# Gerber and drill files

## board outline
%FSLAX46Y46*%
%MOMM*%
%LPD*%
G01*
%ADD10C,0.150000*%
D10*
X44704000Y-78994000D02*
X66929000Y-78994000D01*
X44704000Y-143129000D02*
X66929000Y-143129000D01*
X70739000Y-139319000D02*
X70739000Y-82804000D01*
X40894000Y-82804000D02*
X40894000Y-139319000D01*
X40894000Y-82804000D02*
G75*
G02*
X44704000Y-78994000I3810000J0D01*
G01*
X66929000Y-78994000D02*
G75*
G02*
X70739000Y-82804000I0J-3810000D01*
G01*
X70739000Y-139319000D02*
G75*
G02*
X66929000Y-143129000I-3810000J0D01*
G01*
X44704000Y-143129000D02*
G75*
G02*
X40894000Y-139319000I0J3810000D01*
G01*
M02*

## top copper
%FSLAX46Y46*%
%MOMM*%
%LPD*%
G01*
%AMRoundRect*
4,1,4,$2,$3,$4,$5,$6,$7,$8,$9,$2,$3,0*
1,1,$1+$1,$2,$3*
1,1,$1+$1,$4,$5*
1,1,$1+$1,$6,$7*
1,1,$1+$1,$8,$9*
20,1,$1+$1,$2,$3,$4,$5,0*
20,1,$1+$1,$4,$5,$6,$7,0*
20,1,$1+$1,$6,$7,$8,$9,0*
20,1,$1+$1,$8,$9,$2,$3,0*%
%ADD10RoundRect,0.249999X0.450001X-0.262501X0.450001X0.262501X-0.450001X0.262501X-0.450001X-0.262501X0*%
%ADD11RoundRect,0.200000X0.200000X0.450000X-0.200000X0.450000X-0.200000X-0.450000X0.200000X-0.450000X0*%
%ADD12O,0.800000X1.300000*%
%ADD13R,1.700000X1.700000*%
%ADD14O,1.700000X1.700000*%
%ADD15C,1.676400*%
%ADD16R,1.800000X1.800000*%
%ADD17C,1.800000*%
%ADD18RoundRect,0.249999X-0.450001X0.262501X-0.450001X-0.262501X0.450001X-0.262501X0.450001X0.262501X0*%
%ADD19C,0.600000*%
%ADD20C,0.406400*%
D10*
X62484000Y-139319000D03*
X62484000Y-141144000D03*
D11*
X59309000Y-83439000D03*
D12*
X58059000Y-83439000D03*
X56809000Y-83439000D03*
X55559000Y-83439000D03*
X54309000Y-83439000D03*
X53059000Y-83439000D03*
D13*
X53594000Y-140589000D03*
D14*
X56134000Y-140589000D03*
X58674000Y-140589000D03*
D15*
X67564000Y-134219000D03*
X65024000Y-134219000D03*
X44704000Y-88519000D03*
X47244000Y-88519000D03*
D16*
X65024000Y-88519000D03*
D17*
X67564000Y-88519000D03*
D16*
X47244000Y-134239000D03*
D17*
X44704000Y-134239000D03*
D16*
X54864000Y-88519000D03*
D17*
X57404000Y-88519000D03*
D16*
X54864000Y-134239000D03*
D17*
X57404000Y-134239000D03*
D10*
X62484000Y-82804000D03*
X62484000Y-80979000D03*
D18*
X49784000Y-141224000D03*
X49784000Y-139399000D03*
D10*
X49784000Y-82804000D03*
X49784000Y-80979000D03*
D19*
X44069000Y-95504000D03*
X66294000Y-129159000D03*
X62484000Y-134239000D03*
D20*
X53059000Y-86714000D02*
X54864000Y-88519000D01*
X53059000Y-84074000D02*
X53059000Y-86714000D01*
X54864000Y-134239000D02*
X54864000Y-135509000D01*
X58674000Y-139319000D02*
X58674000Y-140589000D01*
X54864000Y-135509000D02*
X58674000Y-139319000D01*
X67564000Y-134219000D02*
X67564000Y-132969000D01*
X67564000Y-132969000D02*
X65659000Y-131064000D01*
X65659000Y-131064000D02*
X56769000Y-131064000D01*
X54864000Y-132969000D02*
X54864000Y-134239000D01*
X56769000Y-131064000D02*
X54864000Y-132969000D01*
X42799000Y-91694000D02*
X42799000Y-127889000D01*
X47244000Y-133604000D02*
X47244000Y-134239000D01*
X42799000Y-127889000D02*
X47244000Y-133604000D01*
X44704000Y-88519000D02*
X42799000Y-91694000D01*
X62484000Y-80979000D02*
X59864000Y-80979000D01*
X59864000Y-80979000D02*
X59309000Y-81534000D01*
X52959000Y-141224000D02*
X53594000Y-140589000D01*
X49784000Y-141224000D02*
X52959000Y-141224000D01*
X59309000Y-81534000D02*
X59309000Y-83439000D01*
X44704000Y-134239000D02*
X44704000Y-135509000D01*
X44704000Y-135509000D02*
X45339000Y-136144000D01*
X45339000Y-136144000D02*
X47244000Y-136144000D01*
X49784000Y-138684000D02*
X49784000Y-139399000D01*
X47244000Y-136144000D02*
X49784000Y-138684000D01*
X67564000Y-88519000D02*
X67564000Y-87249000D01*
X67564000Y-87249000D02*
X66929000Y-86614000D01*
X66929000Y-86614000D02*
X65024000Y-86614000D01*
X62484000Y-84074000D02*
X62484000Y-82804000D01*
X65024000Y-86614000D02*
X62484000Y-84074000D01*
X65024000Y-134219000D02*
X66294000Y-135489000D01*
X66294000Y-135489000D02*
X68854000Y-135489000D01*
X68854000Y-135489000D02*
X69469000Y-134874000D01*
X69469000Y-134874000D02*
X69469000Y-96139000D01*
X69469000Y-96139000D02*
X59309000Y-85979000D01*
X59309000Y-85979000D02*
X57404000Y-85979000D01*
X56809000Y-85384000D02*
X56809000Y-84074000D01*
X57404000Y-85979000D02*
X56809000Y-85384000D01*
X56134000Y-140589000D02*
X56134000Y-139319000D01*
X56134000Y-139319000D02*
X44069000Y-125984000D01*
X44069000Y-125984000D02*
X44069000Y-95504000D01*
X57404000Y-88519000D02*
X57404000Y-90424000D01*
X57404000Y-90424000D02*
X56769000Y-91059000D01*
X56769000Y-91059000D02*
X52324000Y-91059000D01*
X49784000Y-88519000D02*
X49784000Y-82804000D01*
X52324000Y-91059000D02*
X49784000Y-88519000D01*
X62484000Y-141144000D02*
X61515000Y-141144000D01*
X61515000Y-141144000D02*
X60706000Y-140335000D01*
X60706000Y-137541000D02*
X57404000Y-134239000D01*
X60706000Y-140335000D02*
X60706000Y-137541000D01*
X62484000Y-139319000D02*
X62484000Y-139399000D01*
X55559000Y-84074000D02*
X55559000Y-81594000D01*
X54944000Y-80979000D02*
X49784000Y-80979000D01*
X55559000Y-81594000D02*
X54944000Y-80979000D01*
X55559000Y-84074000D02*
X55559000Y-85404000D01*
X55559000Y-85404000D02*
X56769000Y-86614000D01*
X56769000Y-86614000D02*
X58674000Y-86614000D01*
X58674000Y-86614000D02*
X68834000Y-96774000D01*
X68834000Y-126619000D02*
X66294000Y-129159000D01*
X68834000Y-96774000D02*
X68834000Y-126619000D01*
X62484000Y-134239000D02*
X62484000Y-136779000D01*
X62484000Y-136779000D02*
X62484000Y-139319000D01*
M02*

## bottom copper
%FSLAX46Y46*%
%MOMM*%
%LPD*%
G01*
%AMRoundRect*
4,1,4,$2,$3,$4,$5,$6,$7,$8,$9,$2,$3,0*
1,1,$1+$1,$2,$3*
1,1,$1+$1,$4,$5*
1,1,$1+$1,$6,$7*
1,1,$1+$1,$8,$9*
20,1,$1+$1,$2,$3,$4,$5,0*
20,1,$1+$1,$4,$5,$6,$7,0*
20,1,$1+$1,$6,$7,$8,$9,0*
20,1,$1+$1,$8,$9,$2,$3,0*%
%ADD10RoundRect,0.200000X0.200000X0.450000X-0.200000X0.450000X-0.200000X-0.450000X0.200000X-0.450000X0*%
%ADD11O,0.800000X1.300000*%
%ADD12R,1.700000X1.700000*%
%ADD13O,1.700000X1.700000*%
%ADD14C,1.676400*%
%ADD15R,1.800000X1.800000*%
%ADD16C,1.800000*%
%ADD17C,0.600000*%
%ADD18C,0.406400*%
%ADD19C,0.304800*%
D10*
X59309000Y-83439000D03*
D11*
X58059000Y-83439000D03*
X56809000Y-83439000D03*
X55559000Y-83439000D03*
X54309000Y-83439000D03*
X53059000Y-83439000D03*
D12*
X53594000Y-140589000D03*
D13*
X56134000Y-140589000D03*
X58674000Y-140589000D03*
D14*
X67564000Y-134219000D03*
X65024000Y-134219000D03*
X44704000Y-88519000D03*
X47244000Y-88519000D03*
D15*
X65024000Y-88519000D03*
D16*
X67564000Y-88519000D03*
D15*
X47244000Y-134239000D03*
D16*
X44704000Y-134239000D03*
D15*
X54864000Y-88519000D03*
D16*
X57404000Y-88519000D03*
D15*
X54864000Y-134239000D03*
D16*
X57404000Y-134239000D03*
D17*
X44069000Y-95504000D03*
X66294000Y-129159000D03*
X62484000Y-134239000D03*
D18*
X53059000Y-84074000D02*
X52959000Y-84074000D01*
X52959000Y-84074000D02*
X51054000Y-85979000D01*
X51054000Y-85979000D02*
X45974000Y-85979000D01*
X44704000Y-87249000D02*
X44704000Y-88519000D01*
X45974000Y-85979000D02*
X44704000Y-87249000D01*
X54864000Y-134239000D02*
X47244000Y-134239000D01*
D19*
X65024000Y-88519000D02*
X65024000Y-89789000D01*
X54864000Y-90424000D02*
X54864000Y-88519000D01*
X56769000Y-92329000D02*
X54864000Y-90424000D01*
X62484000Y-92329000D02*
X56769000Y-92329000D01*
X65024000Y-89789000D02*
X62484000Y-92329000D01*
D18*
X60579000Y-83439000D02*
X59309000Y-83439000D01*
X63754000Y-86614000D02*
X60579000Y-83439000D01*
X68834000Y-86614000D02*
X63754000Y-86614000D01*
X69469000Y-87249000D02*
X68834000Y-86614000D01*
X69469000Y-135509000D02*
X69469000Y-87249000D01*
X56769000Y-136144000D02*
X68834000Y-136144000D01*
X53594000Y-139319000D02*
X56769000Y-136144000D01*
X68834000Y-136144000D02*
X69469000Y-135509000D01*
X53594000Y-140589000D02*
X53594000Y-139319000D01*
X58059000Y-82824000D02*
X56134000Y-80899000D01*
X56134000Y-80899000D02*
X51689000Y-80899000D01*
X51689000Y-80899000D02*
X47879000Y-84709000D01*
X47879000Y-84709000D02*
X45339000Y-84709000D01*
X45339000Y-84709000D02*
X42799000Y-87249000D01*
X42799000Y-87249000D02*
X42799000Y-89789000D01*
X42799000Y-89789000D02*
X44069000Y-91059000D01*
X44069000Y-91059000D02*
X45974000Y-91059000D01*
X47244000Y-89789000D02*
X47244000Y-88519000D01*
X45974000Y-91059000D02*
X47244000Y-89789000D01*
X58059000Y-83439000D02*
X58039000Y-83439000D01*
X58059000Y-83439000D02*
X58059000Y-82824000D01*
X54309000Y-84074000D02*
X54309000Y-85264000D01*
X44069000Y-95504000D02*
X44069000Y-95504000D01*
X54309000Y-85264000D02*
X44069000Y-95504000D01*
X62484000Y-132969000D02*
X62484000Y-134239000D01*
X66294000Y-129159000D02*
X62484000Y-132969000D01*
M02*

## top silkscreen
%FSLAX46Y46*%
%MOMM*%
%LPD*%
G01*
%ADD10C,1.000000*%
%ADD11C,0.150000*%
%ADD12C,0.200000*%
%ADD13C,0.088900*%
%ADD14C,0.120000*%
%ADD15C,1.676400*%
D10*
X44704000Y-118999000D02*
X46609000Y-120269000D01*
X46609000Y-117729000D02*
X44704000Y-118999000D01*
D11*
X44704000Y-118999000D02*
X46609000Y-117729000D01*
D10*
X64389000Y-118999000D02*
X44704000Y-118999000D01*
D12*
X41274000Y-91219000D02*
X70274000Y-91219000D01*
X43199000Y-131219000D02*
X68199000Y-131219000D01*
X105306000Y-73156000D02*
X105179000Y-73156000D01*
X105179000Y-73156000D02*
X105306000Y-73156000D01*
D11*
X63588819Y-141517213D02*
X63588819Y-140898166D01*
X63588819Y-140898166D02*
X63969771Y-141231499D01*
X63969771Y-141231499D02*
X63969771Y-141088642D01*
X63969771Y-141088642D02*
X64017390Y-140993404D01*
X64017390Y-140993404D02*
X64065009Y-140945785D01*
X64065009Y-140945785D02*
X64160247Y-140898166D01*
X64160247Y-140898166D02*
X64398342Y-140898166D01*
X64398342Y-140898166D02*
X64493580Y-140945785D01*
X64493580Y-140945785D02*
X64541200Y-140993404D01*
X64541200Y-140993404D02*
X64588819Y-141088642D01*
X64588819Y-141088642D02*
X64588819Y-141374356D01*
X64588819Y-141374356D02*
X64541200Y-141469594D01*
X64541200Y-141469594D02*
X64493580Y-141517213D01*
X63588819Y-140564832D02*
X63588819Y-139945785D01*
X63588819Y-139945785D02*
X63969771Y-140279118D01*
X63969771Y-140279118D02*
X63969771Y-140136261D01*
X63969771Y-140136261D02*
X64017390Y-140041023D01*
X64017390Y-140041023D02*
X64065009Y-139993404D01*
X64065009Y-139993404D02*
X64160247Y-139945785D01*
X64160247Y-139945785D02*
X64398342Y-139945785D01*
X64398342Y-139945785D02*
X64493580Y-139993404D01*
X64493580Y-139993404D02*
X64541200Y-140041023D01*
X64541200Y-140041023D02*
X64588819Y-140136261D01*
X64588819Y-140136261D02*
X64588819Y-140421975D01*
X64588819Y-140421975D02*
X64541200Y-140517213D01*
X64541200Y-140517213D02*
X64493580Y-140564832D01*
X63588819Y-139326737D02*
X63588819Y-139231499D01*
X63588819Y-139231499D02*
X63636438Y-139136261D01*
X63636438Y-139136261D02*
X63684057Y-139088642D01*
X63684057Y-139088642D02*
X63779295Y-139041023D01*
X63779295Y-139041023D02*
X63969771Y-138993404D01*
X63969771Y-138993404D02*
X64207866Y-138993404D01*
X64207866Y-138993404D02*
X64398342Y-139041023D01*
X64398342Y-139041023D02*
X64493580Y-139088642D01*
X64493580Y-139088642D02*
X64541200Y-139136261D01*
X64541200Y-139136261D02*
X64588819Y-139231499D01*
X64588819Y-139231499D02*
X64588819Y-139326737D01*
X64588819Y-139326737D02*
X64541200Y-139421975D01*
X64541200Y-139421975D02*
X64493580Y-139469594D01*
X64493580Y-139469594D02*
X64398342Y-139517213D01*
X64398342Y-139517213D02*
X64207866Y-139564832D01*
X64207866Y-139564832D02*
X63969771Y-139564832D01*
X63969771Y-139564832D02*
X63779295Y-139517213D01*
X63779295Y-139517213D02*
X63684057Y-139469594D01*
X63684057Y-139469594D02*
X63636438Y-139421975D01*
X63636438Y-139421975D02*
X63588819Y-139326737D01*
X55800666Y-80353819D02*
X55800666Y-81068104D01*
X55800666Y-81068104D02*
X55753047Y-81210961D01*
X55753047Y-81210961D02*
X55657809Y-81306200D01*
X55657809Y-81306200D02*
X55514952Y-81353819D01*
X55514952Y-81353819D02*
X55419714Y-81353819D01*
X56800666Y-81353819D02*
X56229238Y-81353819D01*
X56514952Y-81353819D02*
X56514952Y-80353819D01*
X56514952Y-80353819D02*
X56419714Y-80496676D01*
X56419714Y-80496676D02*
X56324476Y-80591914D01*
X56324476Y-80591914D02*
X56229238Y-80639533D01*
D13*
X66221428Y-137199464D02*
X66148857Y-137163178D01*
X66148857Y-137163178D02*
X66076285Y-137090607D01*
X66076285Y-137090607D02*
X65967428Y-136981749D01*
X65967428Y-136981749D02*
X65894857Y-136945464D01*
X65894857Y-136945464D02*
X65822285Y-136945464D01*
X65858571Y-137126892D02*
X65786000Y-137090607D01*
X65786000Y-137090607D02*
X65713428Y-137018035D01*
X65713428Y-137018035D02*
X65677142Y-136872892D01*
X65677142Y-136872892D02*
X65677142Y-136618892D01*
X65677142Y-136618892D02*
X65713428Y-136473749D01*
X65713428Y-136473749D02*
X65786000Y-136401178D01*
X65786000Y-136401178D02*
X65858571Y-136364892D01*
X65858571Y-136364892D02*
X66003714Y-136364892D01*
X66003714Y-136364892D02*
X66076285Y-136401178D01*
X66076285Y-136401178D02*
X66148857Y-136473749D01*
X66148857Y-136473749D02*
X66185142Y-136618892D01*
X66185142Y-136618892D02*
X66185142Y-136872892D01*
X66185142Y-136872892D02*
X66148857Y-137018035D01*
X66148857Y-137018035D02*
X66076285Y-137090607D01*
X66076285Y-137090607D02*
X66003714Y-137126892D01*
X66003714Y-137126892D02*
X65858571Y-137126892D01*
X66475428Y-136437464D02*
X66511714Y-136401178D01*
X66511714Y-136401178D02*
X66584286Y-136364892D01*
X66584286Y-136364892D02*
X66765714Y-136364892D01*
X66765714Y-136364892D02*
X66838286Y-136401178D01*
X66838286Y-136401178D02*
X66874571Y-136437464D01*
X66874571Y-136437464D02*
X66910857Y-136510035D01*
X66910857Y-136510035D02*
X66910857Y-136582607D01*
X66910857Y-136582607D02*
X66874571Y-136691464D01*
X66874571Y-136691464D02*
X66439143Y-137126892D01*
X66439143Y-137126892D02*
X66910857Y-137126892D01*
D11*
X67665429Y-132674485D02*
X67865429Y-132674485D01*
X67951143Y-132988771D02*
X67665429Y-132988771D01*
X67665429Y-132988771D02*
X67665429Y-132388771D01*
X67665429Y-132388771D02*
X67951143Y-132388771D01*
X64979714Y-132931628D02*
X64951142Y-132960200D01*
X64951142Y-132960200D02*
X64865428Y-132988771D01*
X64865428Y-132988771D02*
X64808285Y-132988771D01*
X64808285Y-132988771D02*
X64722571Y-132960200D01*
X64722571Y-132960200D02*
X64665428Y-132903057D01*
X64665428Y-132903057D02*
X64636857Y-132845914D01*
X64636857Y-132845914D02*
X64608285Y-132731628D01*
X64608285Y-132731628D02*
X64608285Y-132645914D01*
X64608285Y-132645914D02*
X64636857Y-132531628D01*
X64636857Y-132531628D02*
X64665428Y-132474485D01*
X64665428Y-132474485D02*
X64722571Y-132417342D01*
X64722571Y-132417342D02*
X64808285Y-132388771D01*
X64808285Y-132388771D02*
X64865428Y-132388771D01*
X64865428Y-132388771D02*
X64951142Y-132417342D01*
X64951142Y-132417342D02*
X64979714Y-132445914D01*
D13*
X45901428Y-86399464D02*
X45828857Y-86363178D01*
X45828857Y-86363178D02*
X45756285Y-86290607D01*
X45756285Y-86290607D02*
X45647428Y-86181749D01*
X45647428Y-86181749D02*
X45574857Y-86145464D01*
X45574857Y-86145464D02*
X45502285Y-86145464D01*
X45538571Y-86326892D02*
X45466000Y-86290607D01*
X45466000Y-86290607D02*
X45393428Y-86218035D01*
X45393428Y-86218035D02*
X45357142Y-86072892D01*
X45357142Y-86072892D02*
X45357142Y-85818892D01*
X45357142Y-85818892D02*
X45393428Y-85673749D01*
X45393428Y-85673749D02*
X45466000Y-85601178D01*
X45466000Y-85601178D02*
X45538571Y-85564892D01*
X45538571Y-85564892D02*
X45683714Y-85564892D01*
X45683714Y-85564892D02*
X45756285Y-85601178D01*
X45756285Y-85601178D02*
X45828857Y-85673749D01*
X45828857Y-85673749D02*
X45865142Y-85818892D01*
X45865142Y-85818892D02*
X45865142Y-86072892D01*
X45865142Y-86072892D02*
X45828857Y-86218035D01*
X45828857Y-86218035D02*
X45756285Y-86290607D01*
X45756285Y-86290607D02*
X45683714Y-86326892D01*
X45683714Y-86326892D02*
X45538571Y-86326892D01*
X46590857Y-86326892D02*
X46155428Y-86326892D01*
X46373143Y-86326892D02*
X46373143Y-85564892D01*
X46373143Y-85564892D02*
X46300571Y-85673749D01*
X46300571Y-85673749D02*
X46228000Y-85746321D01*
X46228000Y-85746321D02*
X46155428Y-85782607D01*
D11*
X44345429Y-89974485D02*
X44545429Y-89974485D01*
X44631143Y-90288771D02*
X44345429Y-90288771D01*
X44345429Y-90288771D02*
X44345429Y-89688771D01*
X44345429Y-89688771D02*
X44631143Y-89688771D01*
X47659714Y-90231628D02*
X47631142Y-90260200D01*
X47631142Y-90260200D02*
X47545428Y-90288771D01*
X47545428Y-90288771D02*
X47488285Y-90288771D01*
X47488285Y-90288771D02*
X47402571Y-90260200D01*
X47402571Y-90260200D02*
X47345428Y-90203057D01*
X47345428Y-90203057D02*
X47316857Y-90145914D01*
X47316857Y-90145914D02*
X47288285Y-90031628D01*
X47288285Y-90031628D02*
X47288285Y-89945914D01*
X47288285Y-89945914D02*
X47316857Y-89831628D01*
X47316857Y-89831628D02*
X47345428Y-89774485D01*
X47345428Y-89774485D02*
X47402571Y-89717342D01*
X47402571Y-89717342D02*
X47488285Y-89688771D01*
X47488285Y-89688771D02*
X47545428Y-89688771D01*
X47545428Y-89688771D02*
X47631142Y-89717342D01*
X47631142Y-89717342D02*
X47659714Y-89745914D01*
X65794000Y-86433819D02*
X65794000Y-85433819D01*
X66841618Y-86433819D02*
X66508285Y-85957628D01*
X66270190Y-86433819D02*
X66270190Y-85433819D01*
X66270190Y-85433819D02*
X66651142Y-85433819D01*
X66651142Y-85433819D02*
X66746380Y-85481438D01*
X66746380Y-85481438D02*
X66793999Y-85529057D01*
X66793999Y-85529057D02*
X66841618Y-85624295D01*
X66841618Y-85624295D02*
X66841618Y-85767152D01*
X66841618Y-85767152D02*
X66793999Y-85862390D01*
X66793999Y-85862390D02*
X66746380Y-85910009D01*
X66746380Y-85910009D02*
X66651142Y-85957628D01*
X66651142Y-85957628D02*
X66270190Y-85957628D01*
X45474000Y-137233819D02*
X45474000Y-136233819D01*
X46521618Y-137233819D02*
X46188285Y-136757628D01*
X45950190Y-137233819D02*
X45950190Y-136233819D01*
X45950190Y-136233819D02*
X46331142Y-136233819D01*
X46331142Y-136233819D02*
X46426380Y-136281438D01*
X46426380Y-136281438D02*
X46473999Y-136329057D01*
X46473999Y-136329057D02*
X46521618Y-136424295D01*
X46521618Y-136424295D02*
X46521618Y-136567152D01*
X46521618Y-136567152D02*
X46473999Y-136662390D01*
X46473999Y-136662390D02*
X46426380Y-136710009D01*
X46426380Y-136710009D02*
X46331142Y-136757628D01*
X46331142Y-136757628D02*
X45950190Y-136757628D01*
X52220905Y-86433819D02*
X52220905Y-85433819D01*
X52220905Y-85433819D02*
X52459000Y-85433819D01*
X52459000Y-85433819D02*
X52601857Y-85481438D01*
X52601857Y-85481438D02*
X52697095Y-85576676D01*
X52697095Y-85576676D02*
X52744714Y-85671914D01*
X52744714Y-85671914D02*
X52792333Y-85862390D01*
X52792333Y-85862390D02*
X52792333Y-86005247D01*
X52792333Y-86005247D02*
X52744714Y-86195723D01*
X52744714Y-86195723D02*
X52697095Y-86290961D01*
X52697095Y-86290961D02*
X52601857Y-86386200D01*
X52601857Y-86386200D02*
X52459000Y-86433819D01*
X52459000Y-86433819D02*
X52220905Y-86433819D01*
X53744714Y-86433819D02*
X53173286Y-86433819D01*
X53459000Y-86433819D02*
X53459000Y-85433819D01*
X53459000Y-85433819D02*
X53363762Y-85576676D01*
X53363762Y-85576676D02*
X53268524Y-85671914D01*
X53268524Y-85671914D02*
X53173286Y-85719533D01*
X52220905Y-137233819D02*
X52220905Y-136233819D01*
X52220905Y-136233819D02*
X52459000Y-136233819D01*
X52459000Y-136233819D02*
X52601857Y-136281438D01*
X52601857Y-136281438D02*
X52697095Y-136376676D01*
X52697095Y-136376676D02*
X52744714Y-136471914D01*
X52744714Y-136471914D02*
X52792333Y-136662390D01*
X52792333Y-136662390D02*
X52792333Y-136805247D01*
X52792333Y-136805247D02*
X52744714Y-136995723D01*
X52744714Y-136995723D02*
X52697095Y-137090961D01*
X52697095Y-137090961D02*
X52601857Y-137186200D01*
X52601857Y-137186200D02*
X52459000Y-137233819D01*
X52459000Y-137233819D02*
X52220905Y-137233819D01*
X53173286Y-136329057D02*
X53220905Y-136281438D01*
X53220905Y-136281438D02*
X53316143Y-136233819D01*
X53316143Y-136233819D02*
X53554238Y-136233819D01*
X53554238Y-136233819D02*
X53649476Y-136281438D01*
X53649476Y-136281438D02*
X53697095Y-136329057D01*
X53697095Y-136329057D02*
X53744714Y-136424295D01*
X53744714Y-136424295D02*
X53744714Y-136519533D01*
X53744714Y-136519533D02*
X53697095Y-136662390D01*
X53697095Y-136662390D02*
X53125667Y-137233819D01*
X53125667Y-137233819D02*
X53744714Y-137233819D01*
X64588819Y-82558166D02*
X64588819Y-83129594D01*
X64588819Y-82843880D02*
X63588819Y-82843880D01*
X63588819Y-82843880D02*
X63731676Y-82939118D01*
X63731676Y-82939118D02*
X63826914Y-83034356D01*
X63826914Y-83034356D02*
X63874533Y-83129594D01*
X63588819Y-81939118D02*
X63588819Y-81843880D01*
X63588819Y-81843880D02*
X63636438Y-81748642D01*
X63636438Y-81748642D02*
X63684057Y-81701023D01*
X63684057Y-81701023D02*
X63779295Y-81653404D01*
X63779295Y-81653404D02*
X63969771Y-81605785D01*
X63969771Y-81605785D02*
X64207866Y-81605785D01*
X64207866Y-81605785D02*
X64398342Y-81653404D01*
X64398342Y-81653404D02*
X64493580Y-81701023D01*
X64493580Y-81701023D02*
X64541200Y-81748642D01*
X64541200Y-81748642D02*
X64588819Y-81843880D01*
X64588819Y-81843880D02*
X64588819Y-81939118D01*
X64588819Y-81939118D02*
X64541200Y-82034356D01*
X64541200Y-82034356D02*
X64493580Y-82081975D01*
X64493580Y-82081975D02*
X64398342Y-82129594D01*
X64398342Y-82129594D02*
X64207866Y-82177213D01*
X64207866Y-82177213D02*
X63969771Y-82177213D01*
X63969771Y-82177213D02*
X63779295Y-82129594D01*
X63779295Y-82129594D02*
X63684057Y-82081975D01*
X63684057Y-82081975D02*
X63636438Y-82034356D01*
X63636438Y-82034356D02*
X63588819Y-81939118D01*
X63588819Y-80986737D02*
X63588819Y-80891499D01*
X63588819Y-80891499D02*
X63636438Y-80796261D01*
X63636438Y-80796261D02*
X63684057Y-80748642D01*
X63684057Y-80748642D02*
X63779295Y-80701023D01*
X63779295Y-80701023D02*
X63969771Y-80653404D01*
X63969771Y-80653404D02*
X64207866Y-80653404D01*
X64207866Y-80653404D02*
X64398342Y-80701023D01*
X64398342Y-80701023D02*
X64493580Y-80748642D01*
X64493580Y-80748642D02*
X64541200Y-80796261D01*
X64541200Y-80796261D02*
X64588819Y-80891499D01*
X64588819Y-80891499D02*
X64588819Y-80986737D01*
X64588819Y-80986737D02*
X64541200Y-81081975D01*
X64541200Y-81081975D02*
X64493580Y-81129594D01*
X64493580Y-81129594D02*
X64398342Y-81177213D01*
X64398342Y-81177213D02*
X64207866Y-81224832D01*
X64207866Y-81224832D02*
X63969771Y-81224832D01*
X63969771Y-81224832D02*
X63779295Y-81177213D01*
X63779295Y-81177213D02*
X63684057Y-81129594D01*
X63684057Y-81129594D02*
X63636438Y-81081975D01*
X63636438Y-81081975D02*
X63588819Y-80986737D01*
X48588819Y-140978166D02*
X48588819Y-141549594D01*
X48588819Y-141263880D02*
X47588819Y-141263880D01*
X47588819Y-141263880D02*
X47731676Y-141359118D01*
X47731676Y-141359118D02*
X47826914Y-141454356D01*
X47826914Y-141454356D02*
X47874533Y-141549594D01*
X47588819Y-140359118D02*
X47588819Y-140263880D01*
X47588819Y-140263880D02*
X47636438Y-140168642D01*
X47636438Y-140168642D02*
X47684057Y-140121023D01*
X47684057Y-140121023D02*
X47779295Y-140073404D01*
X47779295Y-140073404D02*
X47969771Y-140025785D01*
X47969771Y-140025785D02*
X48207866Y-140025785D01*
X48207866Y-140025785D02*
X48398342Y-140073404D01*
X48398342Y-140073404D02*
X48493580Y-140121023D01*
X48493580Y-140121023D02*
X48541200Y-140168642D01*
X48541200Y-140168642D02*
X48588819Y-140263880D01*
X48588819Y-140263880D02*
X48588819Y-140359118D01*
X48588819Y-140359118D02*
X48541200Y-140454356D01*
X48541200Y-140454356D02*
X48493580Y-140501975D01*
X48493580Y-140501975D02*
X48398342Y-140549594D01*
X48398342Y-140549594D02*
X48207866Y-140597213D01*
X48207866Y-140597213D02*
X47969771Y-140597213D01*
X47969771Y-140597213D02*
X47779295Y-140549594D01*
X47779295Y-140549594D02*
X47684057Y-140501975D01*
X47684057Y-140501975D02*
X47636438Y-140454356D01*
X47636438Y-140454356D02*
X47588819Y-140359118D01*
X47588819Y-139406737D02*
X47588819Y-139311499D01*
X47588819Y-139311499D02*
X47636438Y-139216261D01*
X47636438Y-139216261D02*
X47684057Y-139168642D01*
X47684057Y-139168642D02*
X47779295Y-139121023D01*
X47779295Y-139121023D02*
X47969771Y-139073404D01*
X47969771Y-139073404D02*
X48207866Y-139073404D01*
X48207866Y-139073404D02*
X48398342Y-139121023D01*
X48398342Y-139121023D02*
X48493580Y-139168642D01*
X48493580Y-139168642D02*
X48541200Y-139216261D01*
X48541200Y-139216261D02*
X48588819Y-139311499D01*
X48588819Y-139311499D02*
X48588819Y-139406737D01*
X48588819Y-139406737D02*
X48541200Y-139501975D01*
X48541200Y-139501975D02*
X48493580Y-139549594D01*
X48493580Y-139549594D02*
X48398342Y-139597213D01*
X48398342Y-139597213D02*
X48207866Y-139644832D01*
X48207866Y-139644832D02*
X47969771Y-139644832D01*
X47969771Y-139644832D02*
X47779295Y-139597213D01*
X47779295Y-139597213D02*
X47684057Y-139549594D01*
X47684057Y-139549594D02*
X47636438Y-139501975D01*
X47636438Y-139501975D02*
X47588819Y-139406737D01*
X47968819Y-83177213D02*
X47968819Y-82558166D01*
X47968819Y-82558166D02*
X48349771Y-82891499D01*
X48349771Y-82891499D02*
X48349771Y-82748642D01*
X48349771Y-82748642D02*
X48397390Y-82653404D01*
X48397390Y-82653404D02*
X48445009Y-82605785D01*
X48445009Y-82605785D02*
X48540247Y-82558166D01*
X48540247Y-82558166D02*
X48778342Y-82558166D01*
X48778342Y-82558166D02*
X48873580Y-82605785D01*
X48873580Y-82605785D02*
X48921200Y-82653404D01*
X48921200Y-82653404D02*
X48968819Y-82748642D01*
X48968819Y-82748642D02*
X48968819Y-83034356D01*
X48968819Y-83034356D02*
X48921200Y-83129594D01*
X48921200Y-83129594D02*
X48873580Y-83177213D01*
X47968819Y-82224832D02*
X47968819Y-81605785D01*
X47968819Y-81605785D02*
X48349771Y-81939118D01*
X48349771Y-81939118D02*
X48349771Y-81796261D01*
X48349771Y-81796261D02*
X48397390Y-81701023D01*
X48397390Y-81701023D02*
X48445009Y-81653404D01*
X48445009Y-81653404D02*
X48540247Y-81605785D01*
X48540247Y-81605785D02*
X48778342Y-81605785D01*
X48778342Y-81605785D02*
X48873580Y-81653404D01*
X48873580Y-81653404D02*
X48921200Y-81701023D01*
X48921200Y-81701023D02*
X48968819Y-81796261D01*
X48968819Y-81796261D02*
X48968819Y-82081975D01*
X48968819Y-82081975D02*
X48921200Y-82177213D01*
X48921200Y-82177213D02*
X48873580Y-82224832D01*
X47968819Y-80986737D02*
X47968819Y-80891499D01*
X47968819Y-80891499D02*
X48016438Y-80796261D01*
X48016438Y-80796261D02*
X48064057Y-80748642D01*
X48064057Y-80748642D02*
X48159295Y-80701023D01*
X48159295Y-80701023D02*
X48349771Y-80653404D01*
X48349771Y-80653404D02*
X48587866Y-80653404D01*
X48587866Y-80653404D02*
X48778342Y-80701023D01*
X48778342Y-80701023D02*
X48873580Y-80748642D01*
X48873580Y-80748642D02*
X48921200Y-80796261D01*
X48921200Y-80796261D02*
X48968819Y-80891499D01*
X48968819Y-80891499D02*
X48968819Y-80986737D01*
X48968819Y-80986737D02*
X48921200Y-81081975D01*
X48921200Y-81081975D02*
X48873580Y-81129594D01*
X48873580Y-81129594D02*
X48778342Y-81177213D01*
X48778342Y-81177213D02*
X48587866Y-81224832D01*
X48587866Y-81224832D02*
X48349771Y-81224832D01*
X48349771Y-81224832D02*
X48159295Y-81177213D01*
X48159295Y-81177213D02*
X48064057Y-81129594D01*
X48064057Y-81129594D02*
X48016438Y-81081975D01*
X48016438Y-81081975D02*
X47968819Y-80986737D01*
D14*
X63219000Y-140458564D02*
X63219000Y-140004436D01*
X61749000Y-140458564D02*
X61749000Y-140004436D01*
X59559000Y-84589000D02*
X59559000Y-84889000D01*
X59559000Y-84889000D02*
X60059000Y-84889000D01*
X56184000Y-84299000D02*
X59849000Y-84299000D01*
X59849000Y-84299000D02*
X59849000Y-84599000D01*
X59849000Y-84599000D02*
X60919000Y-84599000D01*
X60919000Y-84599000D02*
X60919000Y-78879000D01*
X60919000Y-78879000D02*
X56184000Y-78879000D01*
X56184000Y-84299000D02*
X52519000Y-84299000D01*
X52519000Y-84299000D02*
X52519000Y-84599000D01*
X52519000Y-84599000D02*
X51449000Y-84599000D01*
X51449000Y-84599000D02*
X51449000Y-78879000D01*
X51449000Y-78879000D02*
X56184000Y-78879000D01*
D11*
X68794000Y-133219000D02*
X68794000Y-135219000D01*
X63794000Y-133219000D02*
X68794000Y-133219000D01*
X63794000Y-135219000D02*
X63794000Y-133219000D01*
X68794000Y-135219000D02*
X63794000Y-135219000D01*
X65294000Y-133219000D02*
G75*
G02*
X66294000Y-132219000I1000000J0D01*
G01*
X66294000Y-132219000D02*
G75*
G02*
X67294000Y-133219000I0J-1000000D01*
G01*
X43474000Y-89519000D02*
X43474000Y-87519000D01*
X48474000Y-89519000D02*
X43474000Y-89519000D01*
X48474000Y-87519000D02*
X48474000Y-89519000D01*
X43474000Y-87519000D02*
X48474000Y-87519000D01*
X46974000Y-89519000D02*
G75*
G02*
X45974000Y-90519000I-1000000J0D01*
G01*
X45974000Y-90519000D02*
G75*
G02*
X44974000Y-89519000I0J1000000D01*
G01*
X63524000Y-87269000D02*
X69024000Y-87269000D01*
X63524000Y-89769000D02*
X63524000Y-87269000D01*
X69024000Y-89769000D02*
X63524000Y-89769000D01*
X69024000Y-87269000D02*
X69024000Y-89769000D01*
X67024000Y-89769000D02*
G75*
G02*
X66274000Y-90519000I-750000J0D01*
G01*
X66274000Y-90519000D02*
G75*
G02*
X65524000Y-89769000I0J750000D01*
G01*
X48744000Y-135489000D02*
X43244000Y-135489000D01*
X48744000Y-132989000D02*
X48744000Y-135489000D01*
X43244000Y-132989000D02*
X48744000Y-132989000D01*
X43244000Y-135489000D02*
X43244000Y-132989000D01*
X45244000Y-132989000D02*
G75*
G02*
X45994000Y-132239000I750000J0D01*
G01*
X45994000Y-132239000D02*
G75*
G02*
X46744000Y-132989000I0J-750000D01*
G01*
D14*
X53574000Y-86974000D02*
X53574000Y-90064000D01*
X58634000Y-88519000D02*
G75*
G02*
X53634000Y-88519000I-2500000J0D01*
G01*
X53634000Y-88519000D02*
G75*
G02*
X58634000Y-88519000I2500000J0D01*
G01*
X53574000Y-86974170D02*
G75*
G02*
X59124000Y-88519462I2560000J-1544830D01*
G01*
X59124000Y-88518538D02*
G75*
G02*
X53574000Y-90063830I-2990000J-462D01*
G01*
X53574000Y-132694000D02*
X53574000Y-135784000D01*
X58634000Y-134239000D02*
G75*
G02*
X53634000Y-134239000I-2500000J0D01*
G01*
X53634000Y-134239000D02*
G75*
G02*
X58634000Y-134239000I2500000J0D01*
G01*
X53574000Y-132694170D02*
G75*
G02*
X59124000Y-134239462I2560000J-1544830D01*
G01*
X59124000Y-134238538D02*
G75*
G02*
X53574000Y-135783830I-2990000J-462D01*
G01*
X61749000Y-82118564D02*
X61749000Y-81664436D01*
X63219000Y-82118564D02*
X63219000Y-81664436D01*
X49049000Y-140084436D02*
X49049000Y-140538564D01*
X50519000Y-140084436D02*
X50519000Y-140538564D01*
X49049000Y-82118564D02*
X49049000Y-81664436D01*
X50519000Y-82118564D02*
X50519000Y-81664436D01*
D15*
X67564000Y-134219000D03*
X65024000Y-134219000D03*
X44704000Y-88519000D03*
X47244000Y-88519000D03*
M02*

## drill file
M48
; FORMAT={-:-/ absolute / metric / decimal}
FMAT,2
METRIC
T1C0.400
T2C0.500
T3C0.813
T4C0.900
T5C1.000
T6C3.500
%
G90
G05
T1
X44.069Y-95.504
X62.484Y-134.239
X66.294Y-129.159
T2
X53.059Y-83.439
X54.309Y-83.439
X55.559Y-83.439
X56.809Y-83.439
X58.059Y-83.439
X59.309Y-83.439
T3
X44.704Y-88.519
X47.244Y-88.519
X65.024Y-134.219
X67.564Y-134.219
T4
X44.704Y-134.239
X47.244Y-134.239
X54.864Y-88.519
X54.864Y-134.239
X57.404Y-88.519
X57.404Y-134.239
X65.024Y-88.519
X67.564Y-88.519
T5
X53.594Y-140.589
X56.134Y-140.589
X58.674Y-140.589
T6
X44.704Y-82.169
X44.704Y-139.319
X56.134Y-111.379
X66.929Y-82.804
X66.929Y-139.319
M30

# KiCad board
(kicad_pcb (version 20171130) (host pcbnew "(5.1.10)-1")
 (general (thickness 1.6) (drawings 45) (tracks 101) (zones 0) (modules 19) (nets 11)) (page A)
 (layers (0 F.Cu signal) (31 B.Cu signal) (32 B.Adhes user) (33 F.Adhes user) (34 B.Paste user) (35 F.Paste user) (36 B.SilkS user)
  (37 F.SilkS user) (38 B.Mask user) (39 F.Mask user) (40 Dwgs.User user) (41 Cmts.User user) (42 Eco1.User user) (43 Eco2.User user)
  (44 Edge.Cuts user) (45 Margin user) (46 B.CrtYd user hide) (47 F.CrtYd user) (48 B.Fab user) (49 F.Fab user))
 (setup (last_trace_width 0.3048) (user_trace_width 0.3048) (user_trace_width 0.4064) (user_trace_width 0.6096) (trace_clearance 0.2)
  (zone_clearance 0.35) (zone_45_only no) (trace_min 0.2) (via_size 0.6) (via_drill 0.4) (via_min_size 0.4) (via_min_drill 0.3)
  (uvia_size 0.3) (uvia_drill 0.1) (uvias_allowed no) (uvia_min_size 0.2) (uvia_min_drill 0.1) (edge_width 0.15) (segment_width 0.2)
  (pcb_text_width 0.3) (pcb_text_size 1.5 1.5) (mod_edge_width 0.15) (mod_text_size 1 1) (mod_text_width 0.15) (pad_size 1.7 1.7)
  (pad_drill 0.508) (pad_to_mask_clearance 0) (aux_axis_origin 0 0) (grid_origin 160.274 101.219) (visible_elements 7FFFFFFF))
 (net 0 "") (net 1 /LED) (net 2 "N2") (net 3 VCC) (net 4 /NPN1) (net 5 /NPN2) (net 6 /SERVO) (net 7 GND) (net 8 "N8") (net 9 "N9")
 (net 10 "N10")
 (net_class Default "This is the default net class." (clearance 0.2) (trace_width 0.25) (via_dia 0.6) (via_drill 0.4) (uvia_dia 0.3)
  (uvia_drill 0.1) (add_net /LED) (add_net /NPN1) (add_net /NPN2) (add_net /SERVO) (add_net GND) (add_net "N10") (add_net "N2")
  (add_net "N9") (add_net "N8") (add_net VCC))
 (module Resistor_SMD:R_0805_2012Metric (layer F.Cu) (at 62.484 140.2315 90)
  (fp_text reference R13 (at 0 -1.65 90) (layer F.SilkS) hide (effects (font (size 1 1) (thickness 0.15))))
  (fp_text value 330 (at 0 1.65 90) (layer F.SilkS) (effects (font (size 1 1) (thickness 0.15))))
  (fp_line (start -0.227064 0.735) (end 0.227064 0.735) (layer F.SilkS) (width 0.12))
  (fp_line (start -0.227064 -0.735) (end 0.227064 -0.735) (layer F.SilkS) (width 0.12))
  (pad 2 smd roundrect (at 0.9125 0 90) (size 1.025 1.4) (layers F.Cu F.Paste F.Mask) (roundrect_rratio 0.2439014634146341) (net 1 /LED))
  (pad 1 smd roundrect (at -0.9125 0 90) (size 1.025 1.4) (layers F.Cu F.Paste F.Mask) (roundrect_rratio 0.2439014634146341) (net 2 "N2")))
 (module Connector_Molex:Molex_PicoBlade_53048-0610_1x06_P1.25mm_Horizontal (layer F.Cu) (at 59.309 83.439 180)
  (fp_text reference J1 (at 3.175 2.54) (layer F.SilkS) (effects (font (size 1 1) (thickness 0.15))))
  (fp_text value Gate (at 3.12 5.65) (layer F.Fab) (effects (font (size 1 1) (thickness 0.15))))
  (fp_line (start -0.25 -1.15) (end -0.25 -1.45) (layer F.SilkS) (width 0.12))
  (fp_line (start -0.25 -1.45) (end -0.75 -1.45) (layer F.SilkS) (width 0.12))
  (fp_line (start 3.125 -0.86) (end -0.54 -0.86) (layer F.SilkS) (width 0.12))
  (fp_line (start -0.54 -0.86) (end -0.54 -1.16) (layer F.SilkS) (width 0.12))
  (fp_line (start -0.54 -1.16) (end -1.61 -1.16) (layer F.SilkS) (width 0.12))
  (fp_line (start -1.61 -1.16) (end -1.61 4.56) (layer F.SilkS) (width 0.12))
  (fp_line (start -1.61 4.56) (end 3.125 4.56) (layer F.SilkS) (width 0.12))
  (fp_line (start 3.125 -0.86) (end 6.79 -0.86) (layer F.SilkS) (width 0.12))
  (fp_line (start 6.79 -0.86) (end 6.79 -1.16) (layer F.SilkS) (width 0.12))
  (fp_line (start 6.79 -1.16) (end 7.86 -1.16) (layer F.SilkS) (width 0.12))
  (fp_line (start 7.86 -1.16) (end 7.86 4.56) (layer F.SilkS) (width 0.12))
  (fp_line (start 7.86 4.56) (end 3.125 4.56) (layer F.SilkS) (width 0.12))
  (pad 1 thru_hole roundrect (at 0 0 180) (size 0.8 1.3) (drill 0.5) (layers *.Cu *.Mask) (roundrect_rratio 0.25) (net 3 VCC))
  (pad 2 thru_hole oval (at 1.25 0 180) (size 0.8 1.3) (drill 0.5) (layers *.Cu *.Mask) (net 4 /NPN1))
  (pad 3 thru_hole oval (at 2.5 0 180) (size 0.8 1.3) (drill 0.5) (layers *.Cu *.Mask) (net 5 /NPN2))
  (pad 4 thru_hole oval (at 3.75 0 180) (size 0.8 1.3) (drill 0.5) (layers *.Cu *.Mask) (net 1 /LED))
  (pad 5 thru_hole oval (at 5 0 180) (size 0.8 1.3) (drill 0.5) (layers *.Cu *.Mask) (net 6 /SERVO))
  (pad 6 thru_hole oval (at 6.25 0 180) (size 0.8 1.3) (drill 0.5) (layers *.Cu *.Mask) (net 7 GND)))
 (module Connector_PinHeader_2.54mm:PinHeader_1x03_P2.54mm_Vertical (layer B.Cu) (at 53.594 140.589 270)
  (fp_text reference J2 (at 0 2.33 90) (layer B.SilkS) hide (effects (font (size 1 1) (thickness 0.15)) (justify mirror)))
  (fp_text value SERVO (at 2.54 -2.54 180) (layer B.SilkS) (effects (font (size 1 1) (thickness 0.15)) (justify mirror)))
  (pad 1 thru_hole rect (at 0 0 270) (size 1.7 1.7) (drill 1) (layers *.Cu *.Mask) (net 3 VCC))
  (pad 2 thru_hole oval (at 0 -2.54 270) (size 1.7 1.7) (drill 1) (layers *.Cu *.Mask) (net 6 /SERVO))
  (pad 3 thru_hole oval (at 0 -5.08 270) (size 1.7 1.7) (drill 1) (layers *.Cu *.Mask) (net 7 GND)))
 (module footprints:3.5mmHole (layer F.Cu) (at 66.929 139.319)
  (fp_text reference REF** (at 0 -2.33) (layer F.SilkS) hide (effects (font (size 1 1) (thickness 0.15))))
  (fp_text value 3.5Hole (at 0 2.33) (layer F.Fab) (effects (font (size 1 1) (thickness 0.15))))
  (pad "" np_thru_hole circle (at 0 0) (size 3.5 3.5) (drill 3.5) (layers *.Cu)))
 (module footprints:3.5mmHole (layer F.Cu) (at 66.929 82.804)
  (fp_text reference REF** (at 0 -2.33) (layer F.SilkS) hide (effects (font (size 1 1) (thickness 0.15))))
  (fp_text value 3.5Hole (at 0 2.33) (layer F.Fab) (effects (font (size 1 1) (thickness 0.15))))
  (pad "" np_thru_hole circle (at 0 0) (size 3.5 3.5) (drill 3.5) (layers *.Cu)))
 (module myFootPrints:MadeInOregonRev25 (layer F.Cu) (at 56.134 126.619)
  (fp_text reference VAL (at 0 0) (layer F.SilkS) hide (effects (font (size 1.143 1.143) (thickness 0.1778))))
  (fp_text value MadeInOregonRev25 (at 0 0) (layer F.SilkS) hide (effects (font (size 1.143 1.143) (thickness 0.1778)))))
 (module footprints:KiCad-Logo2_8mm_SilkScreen (layer B.Cu) (at 55.499 120.904 180)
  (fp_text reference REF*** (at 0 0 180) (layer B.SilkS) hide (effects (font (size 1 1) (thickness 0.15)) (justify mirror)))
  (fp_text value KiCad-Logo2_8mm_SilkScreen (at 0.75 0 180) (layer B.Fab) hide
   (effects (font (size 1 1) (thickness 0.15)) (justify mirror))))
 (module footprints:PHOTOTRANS (layer F.Cu) (at 66.294 134.219 180)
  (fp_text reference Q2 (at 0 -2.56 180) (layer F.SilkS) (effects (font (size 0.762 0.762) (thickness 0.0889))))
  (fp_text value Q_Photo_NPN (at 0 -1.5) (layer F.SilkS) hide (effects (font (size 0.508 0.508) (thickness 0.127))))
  (fp_line (start -2.5 1) (end -2.5 -1) (layer F.SilkS) (width 0.15))
  (fp_line (start 2.5 1) (end -2.5 1) (layer F.SilkS) (width 0.15))
  (fp_line (start 2.5 -1) (end 2.5 1) (layer F.SilkS) (width 0.15))
  (fp_line (start -2.5 -1) (end 2.5 -1) (layer F.SilkS) (width 0.15))
  (fp_arc (start 0 1) (end 1 1) (angle 90) (layer F.SilkS) (width 0.15))
  (fp_arc (start 0 1) (end 0 2) (angle 90) (layer F.SilkS) (width 0.15))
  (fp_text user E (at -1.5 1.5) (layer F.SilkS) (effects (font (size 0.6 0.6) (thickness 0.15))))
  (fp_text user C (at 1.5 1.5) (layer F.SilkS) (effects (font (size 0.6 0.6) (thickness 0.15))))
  (pad 2 thru_hole circle (at -1.27 0 180) (size 1.6764 1.6764) (drill 0.8128) (layers *.Cu *.Mask F.SilkS) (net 7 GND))
  (pad 1 thru_hole circle (at 1.27 0 225) (size 1.6764 1.6764) (drill 0.8128) (layers *.Cu *.Mask F.SilkS) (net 5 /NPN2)))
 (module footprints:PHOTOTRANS (layer F.Cu) (at 45.974 88.519)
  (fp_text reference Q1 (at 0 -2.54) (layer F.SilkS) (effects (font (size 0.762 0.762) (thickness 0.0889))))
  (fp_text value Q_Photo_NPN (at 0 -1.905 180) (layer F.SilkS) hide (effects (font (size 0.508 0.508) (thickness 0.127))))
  (fp_line (start -2.5 1) (end -2.5 -1) (layer F.SilkS) (width 0.15))
  (fp_line (start 2.5 1) (end -2.5 1) (layer F.SilkS) (width 0.15))
  (fp_line (start 2.5 -1) (end 2.5 1) (layer F.SilkS) (width 0.15))
  (fp_line (start -2.5 -1) (end 2.5 -1) (layer F.SilkS) (width 0.15))
  (fp_arc (start 0 1) (end 1 1) (angle 90) (layer F.SilkS) (width 0.15))
  (fp_arc (start 0 1) (end 0 2) (angle 90) (layer F.SilkS) (width 0.15))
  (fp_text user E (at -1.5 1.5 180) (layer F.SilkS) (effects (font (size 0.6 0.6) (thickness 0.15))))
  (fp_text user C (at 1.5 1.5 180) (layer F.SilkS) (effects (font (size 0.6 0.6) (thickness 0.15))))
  (pad 2 thru_hole circle (at -1.27 0) (size 1.6764 1.6764) (drill 0.8128) (layers *.Cu *.Mask F.SilkS) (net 7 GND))
  (pad 1 thru_hole circle (at 1.27 0 45) (size 1.6764 1.6764) (drill 0.8128) (layers *.Cu *.Mask F.SilkS) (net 4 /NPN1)))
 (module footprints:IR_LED (layer F.Cu) (at 65.024 88.519)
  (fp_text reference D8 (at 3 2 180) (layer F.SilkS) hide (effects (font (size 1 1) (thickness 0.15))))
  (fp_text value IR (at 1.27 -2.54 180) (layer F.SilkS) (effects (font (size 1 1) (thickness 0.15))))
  (fp_line (start -1.5 -1.25) (end 4 -1.25) (layer F.SilkS) (width 0.15))
  (fp_line (start -1.5 1.25) (end -1.5 -1.25) (layer F.SilkS) (width 0.15))
  (fp_line (start 4 1.25) (end -1.5 1.25) (layer F.SilkS) (width 0.15))
  (fp_line (start 4 -1.25) (end 4 1.25) (layer F.SilkS) (width 0.15))
  (fp_arc (start 1.25 1.25) (end 2 1.25) (angle 90) (layer F.SilkS) (width 0.15))
  (fp_arc (start 1.25 1.25) (end 1.25 2) (angle 90) (layer F.SilkS) (width 0.15))
  (pad 1 thru_hole rect (at 0 0) (size 1.8 1.8) (drill 0.9) (layers *.Cu *.Mask) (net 7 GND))
  (pad 2 thru_hole circle (at 2.54 0) (size 1.8 1.8) (drill 0.9) (layers *.Cu *.Mask) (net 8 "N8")))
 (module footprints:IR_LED (layer F.Cu) (at 47.244 134.239 180)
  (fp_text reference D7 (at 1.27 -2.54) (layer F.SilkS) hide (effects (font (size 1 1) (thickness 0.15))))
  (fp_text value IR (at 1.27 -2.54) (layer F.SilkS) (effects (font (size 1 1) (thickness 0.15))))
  (fp_line (start -1.5 -1.25) (end 4 -1.25) (layer F.SilkS) (width 0.15))
  (fp_line (start -1.5 1.25) (end -1.5 -1.25) (layer F.SilkS) (width 0.15))
  (fp_line (start 4 1.25) (end -1.5 1.25) (layer F.SilkS) (width 0.15))
  (fp_line (start 4 -1.25) (end 4 1.25) (layer F.SilkS) (width 0.15))
  (fp_arc (start 1.25 1.25) (end 2 1.25) (angle 90) (layer F.SilkS) (width 0.15))
  (fp_arc (start 1.25 1.25) (end 1.25 2) (angle 90) (layer F.SilkS) (width 0.15))
  (pad 1 thru_hole rect (at 0 0 180) (size 1.8 1.8) (drill 0.9) (layers *.Cu *.Mask) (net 7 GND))
  (pad 2 thru_hole circle (at 2.54 0 180) (size 1.8 1.8) (drill 0.9) (layers *.Cu *.Mask) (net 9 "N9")))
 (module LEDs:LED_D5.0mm (layer F.Cu) (at 54.864 88.519)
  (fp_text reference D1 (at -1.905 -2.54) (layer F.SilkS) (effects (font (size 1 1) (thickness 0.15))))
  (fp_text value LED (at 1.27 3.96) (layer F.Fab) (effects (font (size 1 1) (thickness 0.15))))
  (fp_line (start -1.29 -1.545) (end -1.29 1.545) (layer F.SilkS) (width 0.12))
  (fp_circle (center 1.27 0) (end 3.77 0) (layer F.SilkS) (width 0.12))
  (fp_arc (start 1.27 0) (end -1.29 -1.54483) (angle 148.9) (layer F.SilkS) (width 0.12))
  (fp_arc (start 1.27 0) (end -1.29 1.54483) (angle -148.9) (layer F.SilkS) (width 0.12))
  (pad 1 thru_hole rect (at 0 0) (size 1.8 1.8) (drill 0.9) (layers *.Cu *.Mask) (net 7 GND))
  (pad 2 thru_hole circle (at 2.54 0) (size 1.8 1.8) (drill 0.9) (layers *.Cu *.Mask) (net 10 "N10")))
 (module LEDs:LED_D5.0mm (layer F.Cu) (at 54.864 134.239)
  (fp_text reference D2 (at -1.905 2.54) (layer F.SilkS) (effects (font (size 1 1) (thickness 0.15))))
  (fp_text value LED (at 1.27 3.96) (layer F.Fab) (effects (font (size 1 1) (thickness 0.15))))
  (fp_line (start -1.29 -1.545) (end -1.29 1.545) (layer F.SilkS) (width 0.12))
  (fp_circle (center 1.27 0) (end 3.77 0) (layer F.SilkS) (width 0.12))
  (fp_arc (start 1.27 0) (end -1.29 -1.54483) (angle 148.9) (layer F.SilkS) (width 0.12))
  (fp_arc (start 1.27 0) (end -1.29 1.54483) (angle -148.9) (layer F.SilkS) (width 0.12))
  (pad 1 thru_hole rect (at 0 0) (size 1.8 1.8) (drill 0.9) (layers *.Cu *.Mask) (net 7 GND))
  (pad 2 thru_hole circle (at 2.54 0) (size 1.8 1.8) (drill 0.9) (layers *.Cu *.Mask) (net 2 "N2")))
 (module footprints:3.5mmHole (layer F.Cu) (at 56.134 111.379)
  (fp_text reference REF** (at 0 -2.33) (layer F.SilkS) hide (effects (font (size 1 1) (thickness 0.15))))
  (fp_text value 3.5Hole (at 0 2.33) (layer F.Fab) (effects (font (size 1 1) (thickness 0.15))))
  (pad "" np_thru_hole circle (at 0 0) (size 3.5 3.5) (drill 3.5) (layers *.Cu)))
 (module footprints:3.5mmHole (layer F.Cu) (at 44.704 139.319)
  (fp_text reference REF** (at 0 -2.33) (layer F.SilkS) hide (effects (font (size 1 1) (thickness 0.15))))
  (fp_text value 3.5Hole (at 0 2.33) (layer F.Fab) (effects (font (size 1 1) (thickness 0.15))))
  (pad "" np_thru_hole circle (at 0 0) (size 3.5 3.5) (drill 3.5) (layers *.Cu)))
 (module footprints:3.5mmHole (layer F.Cu) (at 44.704 82.169)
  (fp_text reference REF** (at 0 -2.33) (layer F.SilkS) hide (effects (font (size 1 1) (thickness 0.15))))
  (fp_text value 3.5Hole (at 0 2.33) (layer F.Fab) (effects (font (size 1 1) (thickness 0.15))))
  (pad "" np_thru_hole circle (at 0 0) (size 3.5 3.5) (drill 3.5) (layers *.Cu)))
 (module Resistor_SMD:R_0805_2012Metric (layer F.Cu) (at 62.484 81.8915 90)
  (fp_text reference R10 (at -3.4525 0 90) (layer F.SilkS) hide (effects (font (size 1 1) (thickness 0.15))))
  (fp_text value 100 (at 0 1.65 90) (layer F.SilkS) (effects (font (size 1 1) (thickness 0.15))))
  (fp_line (start -0.227064 -0.735) (end 0.227064 -0.735) (layer F.SilkS) (width 0.12))
  (fp_line (start -0.227064 0.735) (end 0.227064 0.735) (layer F.SilkS) (width 0.12))
  (pad 1 smd roundrect (at -0.9125 0 90) (size 1.025 1.4) (layers F.Cu F.Paste F.Mask) (roundrect_rratio 0.2439014634146341) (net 8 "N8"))
  (pad 2 smd roundrect (at 0.9125 0 90) (size 1.025 1.4) (layers F.Cu F.Paste F.Mask) (roundrect_rratio 0.2439014634146341) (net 3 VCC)))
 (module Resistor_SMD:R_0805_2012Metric (layer F.Cu) (at 49.784 140.3115 270)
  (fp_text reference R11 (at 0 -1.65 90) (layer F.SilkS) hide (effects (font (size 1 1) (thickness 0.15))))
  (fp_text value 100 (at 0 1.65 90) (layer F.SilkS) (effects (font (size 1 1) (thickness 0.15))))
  (fp_line (start -0.227064 0.735) (end 0.227064 0.735) (layer F.SilkS) (width 0.12))
  (fp_line (start -0.227064 -0.735) (end 0.227064 -0.735) (layer F.SilkS) (width 0.12))
  (pad 2 smd roundrect (at 0.9125 0 270) (size 1.025 1.4) (layers F.Cu F.Paste F.Mask) (roundrect_rratio 0.2439014634146341) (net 3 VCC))
  (pad 1 smd roundrect (at -0.9125 0 270) (size 1.025 1.4) (layers F.Cu F.Paste F.Mask) (roundrect_rratio 0.2439014634146341) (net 9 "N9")))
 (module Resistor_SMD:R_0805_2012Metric (layer F.Cu) (at 49.784 81.8915 90)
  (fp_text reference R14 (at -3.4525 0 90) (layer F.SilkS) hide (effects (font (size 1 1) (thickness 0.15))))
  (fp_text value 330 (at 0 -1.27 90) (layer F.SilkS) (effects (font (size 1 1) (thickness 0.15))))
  (fp_line (start -0.227064 -0.735) (end 0.227064 -0.735) (layer F.SilkS) (width 0.12))
  (fp_line (start -0.227064 0.735) (end 0.227064 0.735) (layer F.SilkS) (width 0.12))
  (pad 1 smd roundrect (at -0.9125 0 90) (size 1.025 1.4) (layers F.Cu F.Paste F.Mask) (roundrect_rratio 0.2439014634146341) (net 10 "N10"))
  (pad 2 smd roundrect (at 0.9125 0 90) (size 1.025 1.4) (layers F.Cu F.Paste F.Mask) (roundrect_rratio 0.2439014634146341) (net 1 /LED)))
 (gr_line (start 44.704 78.994) (end 66.929 78.994) (angle 90) (layer Edge.Cuts) (width 0.15))
 (gr_line (start 44.704 143.129) (end 66.929 143.129) (angle 90) (layer Edge.Cuts) (width 0.15))
 (gr_line (start 70.739 139.319) (end 70.739 82.804) (angle 90) (layer Edge.Cuts) (width 0.15))
 (gr_line (start 40.894 82.804) (end 40.894 139.319) (angle 90) (layer Edge.Cuts) (width 0.15))
 (gr_line (start 44.704 118.999) (end 46.609 120.269) (layer F.SilkS) (width 1))
 (gr_line (start 46.609 117.729) (end 44.704 118.999) (layer F.SilkS) (width 1))
 (gr_line (start 44.704 118.999) (end 46.609 117.729) (layer F.SilkS) (width 0.15))
 (gr_line (start 64.389 118.999) (end 44.704 118.999) (layer F.SilkS) (width 1))
 (gr_arc (start 44.704 82.804) (end 44.704 78.994) (angle -90) (layer Edge.Cuts) (width 0.15))
 (gr_arc (start 66.929 82.804) (end 70.739 82.804) (angle -90) (layer Edge.Cuts) (width 0.15))
 (gr_arc (start 66.929 139.319) (end 66.929 143.129) (angle -90) (layer Edge.Cuts) (width 0.15))
 (gr_arc (start 44.704 139.319) (end 40.894 139.319) (angle -90) (layer Edge.Cuts) (width 0.15))
 (gr_line (start 41.274 91.219) (end 70.274 91.219) (angle 90) (layer F.SilkS) (width 0.2))
 (gr_line (start 43.199 131.219) (end 68.199 131.219) (angle 90) (layer F.SilkS) (width 0.2))
 (gr_line (start 105.306 73.156) (end 105.179 73.156) (angle 90) (layer F.SilkS) (width 0.2))
 (gr_line (start 105.179 73.156) (end 105.306 73.156) (angle 90) (layer F.SilkS) (width 0.2))
 (segment (start 53.059 86.714) (end 54.864 88.519) (width 0.4064) (layer F.Cu) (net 7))
 (segment (start 53.059 84.074) (end 53.059 86.714) (width 0.4064) (layer F.Cu) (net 7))
 (segment (start 53.059 84.074) (end 52.959 84.074) (width 0.4064) (layer B.Cu) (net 7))
 (segment (start 52.959 84.074) (end 51.054 85.979) (width 0.4064) (layer B.Cu) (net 7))
 (segment (start 51.054 85.979) (end 45.974 85.979) (width 0.4064) (layer B.Cu) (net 7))
 (segment (start 44.704 87.249) (end 44.704 88.519) (width 0.4064) (layer B.Cu) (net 7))
 (segment (start 45.974 85.979) (end 44.704 87.249) (width 0.4064) (layer B.Cu) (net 7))
 (segment (start 54.864 134.239) (end 54.864 135.509) (width 0.4064) (layer F.Cu) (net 7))
 (segment (start 58.674 139.319) (end 58.674 140.589) (width 0.4064) (layer F.Cu) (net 7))
 (segment (start 54.864 135.509) (end 58.674 139.319) (width 0.4064) (layer F.Cu) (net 7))
 (segment (start 67.564 134.219) (end 67.564 132.969) (width 0.4064) (layer F.Cu) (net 7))
 (segment (start 67.564 132.969) (end 65.659 131.064) (width 0.4064) (layer F.Cu) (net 7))
 (segment (start 65.659 131.064) (end 56.769 131.064) (width 0.4064) (layer F.Cu) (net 7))
 (segment (start 54.864 132.969) (end 54.864 134.239) (width 0.4064) (layer F.Cu) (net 7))
 (segment (start 56.769 131.064) (end 54.864 132.969) (width 0.4064) (layer F.Cu) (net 7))
 (segment (start 54.864 134.239) (end 47.244 134.239) (width 0.4064) (layer B.Cu) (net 7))
 (segment (start 42.799 91.694) (end 42.799 127.889) (width 0.4064) (layer F.Cu) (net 7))
 (segment (start 47.244 133.604) (end 47.244 134.239) (width 0.4064) (layer F.Cu) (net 7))
 (segment (start 42.799 127.889) (end 47.244 133.604) (width 0.4064) (layer F.Cu) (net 7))
 (segment (start 44.704 88.519) (end 42.799 91.694) (width 0.4064) (layer F.Cu) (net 7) (status 400000))
 (segment (start 65.024 88.519) (end 65.024 89.789) (width 0.3048) (layer B.Cu) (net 7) (status 400000))
 (segment (start 54.864 90.424) (end 54.864 88.519) (width 0.3048) (layer B.Cu) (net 7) (status 800000))
 (segment (start 56.769 92.329) (end 54.864 90.424) (width 0.3048) (layer B.Cu) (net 7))
 (segment (start 62.484 92.329) (end 56.769 92.329) (width 0.3048) (layer B.Cu) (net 7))
 (segment (start 65.024 89.789) (end 62.484 92.329) (width 0.3048) (layer B.Cu) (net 7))
 (segment (start 62.484 80.979) (end 59.864 80.979) (width 0.4064) (layer F.Cu) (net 3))
 (segment (start 59.864 80.979) (end 59.309 81.534) (width 0.4064) (layer F.Cu) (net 3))
 (segment (start 52.959 141.224) (end 53.594 140.589) (width 0.4064) (layer F.Cu) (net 3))
 (segment (start 49.784 141.224) (end 52.959 141.224) (width 0.4064) (layer F.Cu) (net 3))
 (segment (start 59.309 81.534) (end 59.309 83.439) (width 0.4064) (layer F.Cu) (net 3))
 (segment (start 60.579 83.439) (end 59.309 83.439) (width 0.4064) (layer B.Cu) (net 3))
 (segment (start 63.754 86.614) (end 60.579 83.439) (width 0.4064) (layer B.Cu) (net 3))
 (segment (start 68.834 86.614) (end 63.754 86.614) (width 0.4064) (layer B.Cu) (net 3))
 (segment (start 69.469 87.249) (end 68.834 86.614) (width 0.4064) (layer B.Cu) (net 3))
 (segment (start 69.469 135.509) (end 69.469 87.249) (width 0.4064) (layer B.Cu) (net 3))
 (segment (start 56.769 136.144) (end 68.834 136.144) (width 0.4064) (layer B.Cu) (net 3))
 (segment (start 53.594 139.319) (end 56.769 136.144) (width 0.4064) (layer B.Cu) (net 3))
 (segment (start 68.834 136.144) (end 69.469 135.509) (width 0.4064) (layer B.Cu) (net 3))
 (segment (start 53.594 140.589) (end 53.594 139.319) (width 0.4064) (layer B.Cu) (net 3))
 (segment (start 44.704 134.239) (end 44.704 135.509) (width 0.4064) (layer F.Cu) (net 9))
 (segment (start 44.704 135.509) (end 45.339 136.144) (width 0.4064) (layer F.Cu) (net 9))
 (segment (start 45.339 136.144) (end 47.244 136.144) (width 0.4064) (layer F.Cu) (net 9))
 (segment (start 49.784 138.684) (end 49.784 139.399) (width 0.4064) (layer F.Cu) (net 9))
 (segment (start 47.244 136.144) (end 49.784 138.684) (width 0.4064) (layer F.Cu) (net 9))
 (segment (start 67.564 88.519) (end 67.564 87.249) (width 0.4064) (layer F.Cu) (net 8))
 (segment (start 67.564 87.249) (end 66.929 86.614) (width 0.4064) (layer F.Cu) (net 8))
 (segment (start 66.929 86.614) (end 65.024 86.614) (width 0.4064) (layer F.Cu) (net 8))
 (segment (start 62.484 84.074) (end 62.484 82.804) (width 0.4064) (layer F.Cu) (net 8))
 (segment (start 65.024 86.614) (end 62.484 84.074) (width 0.4064) (layer F.Cu) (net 8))
 (segment (start 58.059 82.824) (end 56.134 80.899) (width 0.4064) (layer B.Cu) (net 4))
 (segment (start 56.134 80.899) (end 51.689 80.899) (width 0.4064) (layer B.Cu) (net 4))
 (segment (start 51.689 80.899) (end 47.879 84.709) (width 0.4064) (layer B.Cu) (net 4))
 (segment (start 47.879 84.709) (end 45.339 84.709) (width 0.4064) (layer B.Cu) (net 4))
 (segment (start 45.339 84.709) (end 42.799 87.249) (width 0.4064) (layer B.Cu) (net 4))
 (segment (start 42.799 87.249) (end 42.799 89.789) (width 0.4064) (layer B.Cu) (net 4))
 (segment (start 42.799 89.789) (end 44.069 91.059) (width 0.4064) (layer B.Cu) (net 4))
 (segment (start 44.069 91.059) (end 45.974 91.059) (width 0.4064) (layer B.Cu) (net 4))
 (segment (start 47.244 89.789) (end 47.244 88.519) (width 0.4064) (layer B.Cu) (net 4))
 (segment (start 45.974 91.059) (end 47.244 89.789) (width 0.4064) (layer B.Cu) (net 4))
 (segment (start 58.059 83.439) (end 58.039 83.439) (width 0.4064) (layer B.Cu) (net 4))
 (segment (start 58.059 83.439) (end 58.059 82.824) (width 0.4064) (layer B.Cu) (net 4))
 (segment (start 65.024 134.219) (end 66.294 135.489) (width 0.4064) (layer F.Cu) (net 5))
 (segment (start 66.294 135.489) (end 68.854 135.489) (width 0.4064) (layer F.Cu) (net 5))
 (segment (start 68.854 135.489) (end 69.469 134.874) (width 0.4064) (layer F.Cu) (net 5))
 (segment (start 69.469 134.874) (end 69.469 96.139) (width 0.4064) (layer F.Cu) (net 5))
 (segment (start 69.469 96.139) (end 59.309 85.979) (width 0.4064) (layer F.Cu) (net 5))
 (segment (start 59.309 85.979) (end 57.404 85.979) (width 0.4064) (layer F.Cu) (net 5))
 (segment (start 56.809 85.384) (end 56.809 84.074) (width 0.4064) (layer F.Cu) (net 5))
 (segment (start 57.404 85.979) (end 56.809 85.384) (width 0.4064) (layer F.Cu) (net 5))
 (segment (start 56.134 140.589) (end 56.134 139.319) (width 0.4064) (layer F.Cu) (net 6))
 (segment (start 56.134 139.319) (end 44.069 125.984) (width 0.4064) (layer F.Cu) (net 6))
 (segment (start 44.069 125.984) (end 44.069 95.504) (width 0.4064) (layer F.Cu) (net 6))
 (via (at 44.069 95.504) (size 0.6) (drill 0.4) (layers F.Cu B.Cu) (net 6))
 (segment (start 54.309 84.074) (end 54.309 85.264) (width 0.4064) (layer B.Cu) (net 6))
 (segment (start 44.069 95.504) (end 44.069 95.504) (width 0.4064) (layer B.Cu) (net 6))
 (segment (start 54.309 85.264) (end 44.069 95.504) (width 0.4064) (layer B.Cu) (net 6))
 (segment (start 57.404 88.519) (end 57.404 90.424) (width 0.4064) (layer F.Cu) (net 10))
 (segment (start 57.404 90.424) (end 56.769 91.059) (width 0.4064) (layer F.Cu) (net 10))
 (segment (start 56.769 91.059) (end 52.324 91.059) (width 0.4064) (layer F.Cu) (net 10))
 (segment (start 49.784 88.519) (end 49.784 82.804) (width 0.4064) (layer F.Cu) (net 10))
 (segment (start 52.324 91.059) (end 49.784 88.519) (width 0.4064) (layer F.Cu) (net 10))
 (segment (start 62.484 141.144) (end 61.515 141.144) (width 0.4064) (layer F.Cu) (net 2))
 (segment (start 61.515 141.144) (end 60.706 140.335) (width 0.4064) (layer F.Cu) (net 2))
 (segment (start 60.706 137.541) (end 57.404 134.239) (width 0.4064) (layer F.Cu) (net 2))
 (segment (start 60.706 140.335) (end 60.706 137.541) (width 0.4064) (layer F.Cu) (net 2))
 (segment (start 62.484 139.319) (end 62.484 139.399) (width 0.4064) (layer F.Cu) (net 1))
 (segment (start 55.559 84.074) (end 55.559 81.594) (width 0.4064) (layer F.Cu) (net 1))
 (segment (start 54.944 80.979) (end 49.784 80.979) (width 0.4064) (layer F.Cu) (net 1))
 (segment (start 55.559 81.594) (end 54.944 80.979) (width 0.4064) (layer F.Cu) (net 1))
 (segment (start 55.559 84.074) (end 55.559 85.404) (width 0.4064) (layer F.Cu) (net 1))
 (segment (start 55.559 85.404) (end 56.769 86.614) (width 0.4064) (layer F.Cu) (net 1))
 (segment (start 56.769 86.614) (end 58.674 86.614) (width 0.4064) (layer F.Cu) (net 1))
 (segment (start 58.674 86.614) (end 68.834 96.774) (width 0.4064) (layer F.Cu) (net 1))
 (via (at 66.294 129.159) (size 0.6) (drill 0.4) (layers F.Cu B.Cu) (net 1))
 (segment (start 68.834 126.619) (end 66.294 129.159) (width 0.4064) (layer F.Cu) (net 1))
 (segment (start 68.834 96.774) (end 68.834 126.619) (width 0.4064) (layer F.Cu) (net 1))
 (via (at 62.484 134.239) (size 0.6) (drill 0.4) (layers F.Cu B.Cu) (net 1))
 (segment (start 62.484 132.969) (end 62.484 134.239) (width 0.4064) (layer B.Cu) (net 1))
 (segment (start 66.294 129.159) (end 62.484 132.969) (width 0.4064) (layer B.Cu) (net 1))
 (segment (start 62.484 134.239) (end 62.484 136.779) (width 0.4064) (layer F.Cu) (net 1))
 (segment (start 62.484 136.779) (end 62.484 139.319) (width 0.4064) (layer F.Cu) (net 1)))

